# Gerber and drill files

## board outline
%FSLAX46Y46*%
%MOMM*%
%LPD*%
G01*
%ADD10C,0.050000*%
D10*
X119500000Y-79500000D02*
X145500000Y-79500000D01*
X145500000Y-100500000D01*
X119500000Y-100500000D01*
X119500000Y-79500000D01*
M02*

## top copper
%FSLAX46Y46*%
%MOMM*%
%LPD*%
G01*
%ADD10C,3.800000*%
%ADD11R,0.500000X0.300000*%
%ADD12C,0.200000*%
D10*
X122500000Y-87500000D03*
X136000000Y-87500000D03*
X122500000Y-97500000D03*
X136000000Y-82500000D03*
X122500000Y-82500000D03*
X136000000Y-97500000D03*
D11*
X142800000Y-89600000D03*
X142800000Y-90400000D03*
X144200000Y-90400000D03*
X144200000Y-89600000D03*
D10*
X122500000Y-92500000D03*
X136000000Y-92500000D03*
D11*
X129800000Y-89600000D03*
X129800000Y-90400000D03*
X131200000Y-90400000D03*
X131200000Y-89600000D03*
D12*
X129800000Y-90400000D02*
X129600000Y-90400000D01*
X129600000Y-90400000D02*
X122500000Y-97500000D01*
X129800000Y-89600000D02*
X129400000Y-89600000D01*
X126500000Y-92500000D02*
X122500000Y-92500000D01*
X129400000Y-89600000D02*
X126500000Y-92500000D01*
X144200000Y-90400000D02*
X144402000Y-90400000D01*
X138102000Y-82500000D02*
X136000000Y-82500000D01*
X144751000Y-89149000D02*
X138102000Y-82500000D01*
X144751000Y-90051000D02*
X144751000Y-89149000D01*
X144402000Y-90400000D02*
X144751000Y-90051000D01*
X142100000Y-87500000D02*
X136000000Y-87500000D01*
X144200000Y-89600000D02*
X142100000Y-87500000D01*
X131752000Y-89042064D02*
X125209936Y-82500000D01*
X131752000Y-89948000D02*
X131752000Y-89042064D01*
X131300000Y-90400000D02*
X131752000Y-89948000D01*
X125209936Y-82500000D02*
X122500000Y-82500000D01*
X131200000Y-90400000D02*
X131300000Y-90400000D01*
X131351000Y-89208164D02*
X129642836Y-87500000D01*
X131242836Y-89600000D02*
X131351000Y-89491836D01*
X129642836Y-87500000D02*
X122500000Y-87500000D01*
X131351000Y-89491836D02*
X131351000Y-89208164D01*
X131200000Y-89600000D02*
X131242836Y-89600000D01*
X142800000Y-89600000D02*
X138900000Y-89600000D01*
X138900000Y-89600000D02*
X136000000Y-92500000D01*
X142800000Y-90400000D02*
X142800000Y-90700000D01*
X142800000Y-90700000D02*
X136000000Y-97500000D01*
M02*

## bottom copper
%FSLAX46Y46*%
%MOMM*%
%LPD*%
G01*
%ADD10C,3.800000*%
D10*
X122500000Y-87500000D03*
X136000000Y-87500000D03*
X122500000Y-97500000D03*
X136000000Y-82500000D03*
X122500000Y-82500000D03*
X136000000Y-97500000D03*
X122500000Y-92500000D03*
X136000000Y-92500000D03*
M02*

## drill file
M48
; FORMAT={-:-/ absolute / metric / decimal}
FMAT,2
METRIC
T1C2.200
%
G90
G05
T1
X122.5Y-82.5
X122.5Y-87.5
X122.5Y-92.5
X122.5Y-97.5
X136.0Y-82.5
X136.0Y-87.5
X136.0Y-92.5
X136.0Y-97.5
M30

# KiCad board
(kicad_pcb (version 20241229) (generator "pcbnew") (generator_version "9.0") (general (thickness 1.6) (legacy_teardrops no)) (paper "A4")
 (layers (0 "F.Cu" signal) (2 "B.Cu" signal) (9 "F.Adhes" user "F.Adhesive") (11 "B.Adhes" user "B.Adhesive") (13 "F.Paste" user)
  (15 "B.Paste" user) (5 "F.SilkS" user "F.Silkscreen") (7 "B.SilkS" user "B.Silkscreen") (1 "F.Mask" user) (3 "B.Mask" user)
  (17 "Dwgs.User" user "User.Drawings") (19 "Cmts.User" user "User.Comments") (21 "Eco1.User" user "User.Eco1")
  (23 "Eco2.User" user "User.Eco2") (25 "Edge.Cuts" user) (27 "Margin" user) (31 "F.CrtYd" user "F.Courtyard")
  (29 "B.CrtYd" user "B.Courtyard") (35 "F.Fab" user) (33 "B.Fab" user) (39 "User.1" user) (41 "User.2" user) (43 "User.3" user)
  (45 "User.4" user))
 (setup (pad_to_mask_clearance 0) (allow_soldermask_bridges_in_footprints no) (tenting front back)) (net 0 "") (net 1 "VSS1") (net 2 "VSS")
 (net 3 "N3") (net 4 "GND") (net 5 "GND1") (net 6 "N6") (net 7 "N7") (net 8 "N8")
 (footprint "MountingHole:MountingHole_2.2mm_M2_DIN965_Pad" (layer "F.Cu") (at 122.5 87.5)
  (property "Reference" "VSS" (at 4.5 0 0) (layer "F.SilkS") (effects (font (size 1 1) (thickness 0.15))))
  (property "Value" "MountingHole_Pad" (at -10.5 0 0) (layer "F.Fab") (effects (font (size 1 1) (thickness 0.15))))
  (pad "1" thru_hole circle (at 0 0) (size 3.8 3.8) (drill 2.2) (layers "*.Cu" "*.Mask") (remove_unused_layers no) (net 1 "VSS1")
   (zone_connect 2)))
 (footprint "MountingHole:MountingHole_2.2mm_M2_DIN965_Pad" (layer "F.Cu") (at 136 87.5)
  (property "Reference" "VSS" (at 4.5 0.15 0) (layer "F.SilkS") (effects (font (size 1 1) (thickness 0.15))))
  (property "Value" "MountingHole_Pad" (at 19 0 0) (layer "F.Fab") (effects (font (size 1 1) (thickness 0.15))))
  (pad "1" thru_hole circle (at 0 0) (size 3.8 3.8) (drill 2.2) (layers "*.Cu" "*.Mask") (remove_unused_layers no) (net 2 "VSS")
   (zone_connect 2)))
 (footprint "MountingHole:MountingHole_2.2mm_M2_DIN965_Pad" (layer "F.Cu") (at 122.5 97.5)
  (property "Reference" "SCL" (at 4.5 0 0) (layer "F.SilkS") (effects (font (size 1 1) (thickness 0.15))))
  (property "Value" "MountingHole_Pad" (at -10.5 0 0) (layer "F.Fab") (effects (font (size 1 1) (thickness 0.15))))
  (pad "1" thru_hole circle (at 0 0) (size 3.8 3.8) (drill 2.2) (layers "*.Cu" "*.Mask") (remove_unused_layers no) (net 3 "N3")
   (zone_connect 2)))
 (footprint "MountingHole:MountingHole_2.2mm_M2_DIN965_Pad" (layer "F.Cu") (at 136 82.5)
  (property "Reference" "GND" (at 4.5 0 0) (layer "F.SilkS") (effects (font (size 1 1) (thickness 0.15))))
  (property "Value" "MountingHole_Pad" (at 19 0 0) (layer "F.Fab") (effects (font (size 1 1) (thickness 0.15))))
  (pad "1" thru_hole circle (at 0 0) (size 3.8 3.8) (drill 2.2) (layers "*.Cu" "*.Mask") (remove_unused_layers no) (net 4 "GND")
   (zone_connect 2)))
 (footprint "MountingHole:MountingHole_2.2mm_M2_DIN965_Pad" (layer "F.Cu") (at 122.5 82.5)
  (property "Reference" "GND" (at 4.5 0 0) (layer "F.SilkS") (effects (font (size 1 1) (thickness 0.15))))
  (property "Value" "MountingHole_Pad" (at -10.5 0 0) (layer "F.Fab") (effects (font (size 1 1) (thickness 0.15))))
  (pad "1" thru_hole circle (at 0 0) (size 3.8 3.8) (drill 2.2) (layers "*.Cu" "*.Mask") (remove_unused_layers no) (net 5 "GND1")
   (zone_connect 2)))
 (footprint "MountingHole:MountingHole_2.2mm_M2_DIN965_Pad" (layer "F.Cu") (at 136 97.5)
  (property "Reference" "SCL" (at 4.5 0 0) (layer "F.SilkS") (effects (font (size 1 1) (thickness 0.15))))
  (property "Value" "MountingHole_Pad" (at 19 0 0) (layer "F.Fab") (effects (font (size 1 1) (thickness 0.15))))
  (pad "1" thru_hole circle (at 0 0) (size 3.8 3.8) (drill 2.2) (layers "*.Cu" "*.Mask") (remove_unused_layers no) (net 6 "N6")
   (zone_connect 2)))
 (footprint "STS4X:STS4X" (layer "F.Cu") (at 143.5 90)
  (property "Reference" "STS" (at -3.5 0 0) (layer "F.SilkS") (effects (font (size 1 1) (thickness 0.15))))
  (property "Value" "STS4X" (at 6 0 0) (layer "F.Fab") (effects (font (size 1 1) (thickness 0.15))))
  (pad "1" smd rect (at -0.7 -0.4) (size 0.5 0.3) (layers "F.Cu" "F.Mask" "F.Paste") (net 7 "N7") (solder_mask_margin 0.102))
  (pad "2" smd rect (at -0.7 0.4) (size 0.5 0.3) (layers "F.Cu" "F.Mask" "F.Paste") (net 6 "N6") (solder_mask_margin 0.102))
  (pad "3" smd rect (at 0.7 0.4) (size 0.5 0.3) (layers "F.Cu" "F.Mask" "F.Paste") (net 4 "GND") (solder_mask_margin 0.102))
  (pad "4" smd rect (at 0.7 -0.4) (size 0.5 0.3) (layers "F.Cu" "F.Mask" "F.Paste") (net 2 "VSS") (solder_mask_margin 0.102)))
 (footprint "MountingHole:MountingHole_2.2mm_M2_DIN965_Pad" (layer "F.Cu") (at 122.5 92.5)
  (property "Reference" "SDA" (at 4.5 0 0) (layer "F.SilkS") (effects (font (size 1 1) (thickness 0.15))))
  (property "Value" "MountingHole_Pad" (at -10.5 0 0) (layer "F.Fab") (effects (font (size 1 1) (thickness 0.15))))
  (pad "1" thru_hole circle (at 0 0) (size 3.8 3.8) (drill 2.2) (layers "*.Cu" "*.Mask") (remove_unused_layers no) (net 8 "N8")
   (zone_connect 2)))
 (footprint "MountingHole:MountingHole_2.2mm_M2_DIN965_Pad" (layer "F.Cu") (at 136 92.5)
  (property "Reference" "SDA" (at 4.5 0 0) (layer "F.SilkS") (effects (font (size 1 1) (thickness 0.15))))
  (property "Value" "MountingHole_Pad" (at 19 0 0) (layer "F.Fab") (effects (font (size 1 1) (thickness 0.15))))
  (pad "1" thru_hole circle (at 0 0) (size 3.8 3.8) (drill 2.2) (layers "*.Cu" "*.Mask") (remove_unused_layers no) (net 7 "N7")
   (zone_connect 2)))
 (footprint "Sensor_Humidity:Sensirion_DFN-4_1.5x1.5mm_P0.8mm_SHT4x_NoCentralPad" (layer "F.Cu") (at 130.5 90)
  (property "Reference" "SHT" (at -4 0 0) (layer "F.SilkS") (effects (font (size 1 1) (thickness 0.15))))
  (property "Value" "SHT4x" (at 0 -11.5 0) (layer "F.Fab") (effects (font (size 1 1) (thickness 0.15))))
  (pad "1" smd rect (at -0.7 -0.4) (size 0.5 0.3) (layers "F.Cu" "F.Mask" "F.Paste") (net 8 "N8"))
  (pad "2" smd rect (at -0.7 0.4) (size 0.5 0.3) (layers "F.Cu" "F.Mask" "F.Paste") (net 3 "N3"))
  (pad "3" smd rect (at 0.7 0.4) (size 0.5 0.3) (layers "F.Cu" "F.Mask" "F.Paste") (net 5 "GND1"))
  (pad "4" smd rect (at 0.7 -0.4) (size 0.5 0.3) (layers "F.Cu" "F.Mask" "F.Paste") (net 1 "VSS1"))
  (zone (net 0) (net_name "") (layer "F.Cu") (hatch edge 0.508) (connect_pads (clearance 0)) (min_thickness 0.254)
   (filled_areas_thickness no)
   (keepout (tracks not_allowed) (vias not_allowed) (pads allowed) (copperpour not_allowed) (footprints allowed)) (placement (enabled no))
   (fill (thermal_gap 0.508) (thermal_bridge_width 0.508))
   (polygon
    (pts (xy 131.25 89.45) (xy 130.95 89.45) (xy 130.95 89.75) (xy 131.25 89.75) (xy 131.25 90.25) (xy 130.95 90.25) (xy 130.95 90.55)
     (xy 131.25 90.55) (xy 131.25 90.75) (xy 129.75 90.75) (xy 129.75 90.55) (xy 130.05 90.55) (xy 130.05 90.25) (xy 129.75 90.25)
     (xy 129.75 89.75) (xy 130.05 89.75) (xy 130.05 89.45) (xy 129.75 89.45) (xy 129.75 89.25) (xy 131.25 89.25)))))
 (gr_rect (start 119.5 79.5) (end 145.5 100.5) (stroke (width 0.05) (type default)) (fill no) (layer "Edge.Cuts"))
 (segment (start 129.8 90.4) (end 129.6 90.4) (width 0.2) (layer "F.Cu") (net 3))
 (segment (start 129.6 90.4) (end 122.5 97.5) (width 0.2) (layer "F.Cu") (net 3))
 (segment (start 129.8 89.6) (end 129.4 89.6) (width 0.2) (layer "F.Cu") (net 8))
 (segment (start 126.5 92.5) (end 122.5 92.5) (width 0.2) (layer "F.Cu") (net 8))
 (segment (start 129.4 89.6) (end 126.5 92.5) (width 0.2) (layer "F.Cu") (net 8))
 (segment (start 144.2 90.4) (end 144.402 90.4) (width 0.2) (layer "F.Cu") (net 4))
 (segment (start 138.102 82.5) (end 136 82.5) (width 0.2) (layer "F.Cu") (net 4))
 (segment (start 144.751 89.149) (end 138.102 82.5) (width 0.2) (layer "F.Cu") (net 4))
 (segment (start 144.751 90.051) (end 144.751 89.149) (width 0.2) (layer "F.Cu") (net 4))
 (segment (start 144.402 90.4) (end 144.751 90.051) (width 0.2) (layer "F.Cu") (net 4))
 (segment (start 142.1 87.5) (end 136 87.5) (width 0.2) (layer "F.Cu") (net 2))
 (segment (start 144.2 89.6) (end 142.1 87.5) (width 0.2) (layer "F.Cu") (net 2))
 (segment (start 131.752 89.042064) (end 125.209936 82.5) (width 0.2) (layer "F.Cu") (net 5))
 (segment (start 131.752 89.948) (end 131.752 89.042064) (width 0.2) (layer "F.Cu") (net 5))
 (segment (start 131.3 90.4) (end 131.752 89.948) (width 0.2) (layer "F.Cu") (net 5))
 (segment (start 125.209936 82.5) (end 122.5 82.5) (width 0.2) (layer "F.Cu") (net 5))
 (segment (start 131.2 90.4) (end 131.3 90.4) (width 0.2) (layer "F.Cu") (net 5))
 (segment (start 131.351 89.208164) (end 129.642836 87.5) (width 0.2) (layer "F.Cu") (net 1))
 (segment (start 131.242836 89.6) (end 131.351 89.491836) (width 0.2) (layer "F.Cu") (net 1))
 (segment (start 129.642836 87.5) (end 122.5 87.5) (width 0.2) (layer "F.Cu") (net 1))
 (segment (start 131.351 89.491836) (end 131.351 89.208164) (width 0.2) (layer "F.Cu") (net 1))
 (segment (start 131.2 89.6) (end 131.242836 89.6) (width 0.2) (layer "F.Cu") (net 1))
 (segment (start 142.8 89.6) (end 138.9 89.6) (width 0.2) (layer "F.Cu") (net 7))
 (segment (start 138.9 89.6) (end 136 92.5) (width 0.2) (layer "F.Cu") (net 7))
 (segment (start 142.8 90.4) (end 142.8 90.7) (width 0.2) (layer "F.Cu") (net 6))
 (segment (start 142.8 90.7) (end 136 97.5) (width 0.2) (layer "F.Cu") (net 6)))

